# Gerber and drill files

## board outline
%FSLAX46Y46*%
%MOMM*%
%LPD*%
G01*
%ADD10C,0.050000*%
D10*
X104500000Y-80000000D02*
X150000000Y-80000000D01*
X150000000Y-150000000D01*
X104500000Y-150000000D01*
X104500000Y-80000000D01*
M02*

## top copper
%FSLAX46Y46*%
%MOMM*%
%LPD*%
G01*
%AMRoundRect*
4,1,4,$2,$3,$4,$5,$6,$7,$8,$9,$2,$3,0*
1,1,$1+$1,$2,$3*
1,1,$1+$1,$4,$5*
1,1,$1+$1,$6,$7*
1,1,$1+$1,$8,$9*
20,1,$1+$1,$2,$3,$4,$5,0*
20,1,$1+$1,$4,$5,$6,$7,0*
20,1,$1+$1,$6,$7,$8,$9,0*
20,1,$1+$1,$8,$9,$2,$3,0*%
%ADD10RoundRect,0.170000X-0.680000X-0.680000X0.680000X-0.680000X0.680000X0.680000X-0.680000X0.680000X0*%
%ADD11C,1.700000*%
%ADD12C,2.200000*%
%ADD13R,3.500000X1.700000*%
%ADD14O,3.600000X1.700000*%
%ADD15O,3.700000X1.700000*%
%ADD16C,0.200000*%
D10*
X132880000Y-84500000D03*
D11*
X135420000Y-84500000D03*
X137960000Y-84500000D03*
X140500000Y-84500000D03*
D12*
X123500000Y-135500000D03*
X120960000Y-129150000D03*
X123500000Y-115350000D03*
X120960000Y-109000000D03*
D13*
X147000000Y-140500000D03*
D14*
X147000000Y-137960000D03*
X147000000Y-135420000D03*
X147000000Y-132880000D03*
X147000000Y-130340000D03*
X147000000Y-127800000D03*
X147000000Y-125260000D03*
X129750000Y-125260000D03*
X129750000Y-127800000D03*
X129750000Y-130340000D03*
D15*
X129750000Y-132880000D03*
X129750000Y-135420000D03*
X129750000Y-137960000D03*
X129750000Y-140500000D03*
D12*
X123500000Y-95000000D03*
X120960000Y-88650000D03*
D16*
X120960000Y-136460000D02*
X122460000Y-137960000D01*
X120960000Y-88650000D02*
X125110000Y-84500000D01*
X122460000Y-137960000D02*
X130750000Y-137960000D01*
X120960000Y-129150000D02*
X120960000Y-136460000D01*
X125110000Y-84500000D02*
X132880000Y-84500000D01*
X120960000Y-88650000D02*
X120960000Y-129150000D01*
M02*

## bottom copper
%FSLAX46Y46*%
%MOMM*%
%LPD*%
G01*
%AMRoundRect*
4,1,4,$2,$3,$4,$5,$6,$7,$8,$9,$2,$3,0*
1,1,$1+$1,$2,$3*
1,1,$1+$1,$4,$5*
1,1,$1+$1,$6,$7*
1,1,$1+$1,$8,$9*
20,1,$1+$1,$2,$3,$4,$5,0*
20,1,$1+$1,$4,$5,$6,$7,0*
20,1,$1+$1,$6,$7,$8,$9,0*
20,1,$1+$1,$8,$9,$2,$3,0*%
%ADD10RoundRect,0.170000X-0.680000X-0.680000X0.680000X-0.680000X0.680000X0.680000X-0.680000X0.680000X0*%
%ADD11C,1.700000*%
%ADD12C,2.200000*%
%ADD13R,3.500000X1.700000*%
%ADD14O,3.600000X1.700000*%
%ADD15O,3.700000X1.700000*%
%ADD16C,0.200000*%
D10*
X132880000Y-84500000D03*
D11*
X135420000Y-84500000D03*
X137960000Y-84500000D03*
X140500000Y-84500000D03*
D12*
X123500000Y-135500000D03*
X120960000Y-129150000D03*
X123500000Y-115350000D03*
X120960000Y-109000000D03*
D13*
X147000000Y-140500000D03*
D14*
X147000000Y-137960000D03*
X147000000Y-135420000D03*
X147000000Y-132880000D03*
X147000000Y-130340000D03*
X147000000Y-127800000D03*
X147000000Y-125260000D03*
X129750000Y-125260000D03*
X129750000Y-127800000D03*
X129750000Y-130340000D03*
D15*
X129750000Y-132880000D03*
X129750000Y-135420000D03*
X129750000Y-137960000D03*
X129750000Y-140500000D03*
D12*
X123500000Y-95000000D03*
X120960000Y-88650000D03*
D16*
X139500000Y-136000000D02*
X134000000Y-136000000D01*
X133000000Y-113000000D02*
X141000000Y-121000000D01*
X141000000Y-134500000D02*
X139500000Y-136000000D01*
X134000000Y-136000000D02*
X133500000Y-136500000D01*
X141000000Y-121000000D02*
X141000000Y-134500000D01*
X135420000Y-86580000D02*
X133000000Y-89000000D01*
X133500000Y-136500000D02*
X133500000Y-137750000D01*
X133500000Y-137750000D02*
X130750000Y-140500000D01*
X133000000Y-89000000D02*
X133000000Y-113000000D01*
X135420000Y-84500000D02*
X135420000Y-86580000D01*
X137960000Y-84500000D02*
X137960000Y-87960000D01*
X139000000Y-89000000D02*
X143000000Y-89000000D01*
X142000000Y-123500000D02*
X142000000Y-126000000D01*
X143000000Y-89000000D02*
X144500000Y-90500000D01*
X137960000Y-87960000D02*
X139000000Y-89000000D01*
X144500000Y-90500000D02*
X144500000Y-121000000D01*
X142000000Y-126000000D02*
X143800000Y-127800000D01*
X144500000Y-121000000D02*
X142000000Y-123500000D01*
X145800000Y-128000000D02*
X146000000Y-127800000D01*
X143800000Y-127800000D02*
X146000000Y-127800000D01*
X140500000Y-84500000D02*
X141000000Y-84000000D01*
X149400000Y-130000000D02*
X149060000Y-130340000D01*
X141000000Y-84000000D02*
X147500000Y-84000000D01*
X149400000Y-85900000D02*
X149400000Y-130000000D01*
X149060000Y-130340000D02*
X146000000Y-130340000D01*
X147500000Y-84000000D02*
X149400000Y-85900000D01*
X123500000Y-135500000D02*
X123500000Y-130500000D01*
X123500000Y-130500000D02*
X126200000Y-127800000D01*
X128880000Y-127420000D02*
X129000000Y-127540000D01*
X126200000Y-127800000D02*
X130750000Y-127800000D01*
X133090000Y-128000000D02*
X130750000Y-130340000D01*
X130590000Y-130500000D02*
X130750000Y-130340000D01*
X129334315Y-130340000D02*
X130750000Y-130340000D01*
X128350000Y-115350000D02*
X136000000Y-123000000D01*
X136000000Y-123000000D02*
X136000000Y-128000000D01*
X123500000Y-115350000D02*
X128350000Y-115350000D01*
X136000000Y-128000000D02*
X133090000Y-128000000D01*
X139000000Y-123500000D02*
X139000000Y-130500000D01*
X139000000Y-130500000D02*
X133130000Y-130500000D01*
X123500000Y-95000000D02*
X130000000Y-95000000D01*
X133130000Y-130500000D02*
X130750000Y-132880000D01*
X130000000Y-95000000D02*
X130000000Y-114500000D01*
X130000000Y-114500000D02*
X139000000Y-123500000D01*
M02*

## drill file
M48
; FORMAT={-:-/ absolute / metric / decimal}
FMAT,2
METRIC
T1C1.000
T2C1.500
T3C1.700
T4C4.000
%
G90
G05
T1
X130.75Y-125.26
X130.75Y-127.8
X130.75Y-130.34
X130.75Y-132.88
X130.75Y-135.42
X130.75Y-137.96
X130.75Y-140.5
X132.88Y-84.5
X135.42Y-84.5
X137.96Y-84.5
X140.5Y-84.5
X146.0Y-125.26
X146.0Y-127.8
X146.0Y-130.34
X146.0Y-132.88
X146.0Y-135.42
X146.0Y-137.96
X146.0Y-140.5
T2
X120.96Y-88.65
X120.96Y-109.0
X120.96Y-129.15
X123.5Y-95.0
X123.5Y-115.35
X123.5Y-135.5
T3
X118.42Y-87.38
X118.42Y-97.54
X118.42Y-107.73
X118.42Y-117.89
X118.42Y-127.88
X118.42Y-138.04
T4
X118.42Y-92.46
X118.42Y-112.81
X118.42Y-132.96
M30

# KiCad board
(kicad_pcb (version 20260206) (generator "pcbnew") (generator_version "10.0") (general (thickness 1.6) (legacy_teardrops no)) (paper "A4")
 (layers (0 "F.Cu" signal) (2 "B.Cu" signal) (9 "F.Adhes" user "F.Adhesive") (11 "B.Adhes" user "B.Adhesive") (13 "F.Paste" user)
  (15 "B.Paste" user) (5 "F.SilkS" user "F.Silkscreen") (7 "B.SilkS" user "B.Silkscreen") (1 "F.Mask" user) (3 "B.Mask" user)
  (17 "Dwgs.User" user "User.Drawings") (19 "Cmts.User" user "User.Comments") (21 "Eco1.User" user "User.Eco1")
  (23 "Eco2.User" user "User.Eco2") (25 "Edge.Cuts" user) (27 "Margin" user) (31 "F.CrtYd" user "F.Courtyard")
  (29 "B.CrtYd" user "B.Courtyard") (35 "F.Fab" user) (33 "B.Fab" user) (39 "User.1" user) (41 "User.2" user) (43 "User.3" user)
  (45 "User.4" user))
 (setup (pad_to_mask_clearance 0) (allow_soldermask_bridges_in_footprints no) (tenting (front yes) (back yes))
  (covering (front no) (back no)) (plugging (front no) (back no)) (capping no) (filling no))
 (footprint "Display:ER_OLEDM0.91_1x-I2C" (layer "F.Cu") (at 132.88 84.5)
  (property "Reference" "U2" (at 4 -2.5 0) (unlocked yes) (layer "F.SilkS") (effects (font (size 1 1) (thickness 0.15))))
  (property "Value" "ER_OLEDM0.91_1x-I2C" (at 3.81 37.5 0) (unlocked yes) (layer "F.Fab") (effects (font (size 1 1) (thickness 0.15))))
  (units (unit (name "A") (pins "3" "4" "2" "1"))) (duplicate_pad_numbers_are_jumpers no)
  (pad "1" thru_hole roundrect (at 0 0) (size 1.7 1.7) (drill 1) (layers "*.Cu" "*.Mask") (remove_unused_layers no) (roundrect_rratio 0.1)
   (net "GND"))
  (pad "2" thru_hole circle (at 2.54 0) (size 1.7 1.7) (drill 1) (layers "*.Cu" "*.Mask") (remove_unused_layers no) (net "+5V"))
  (pad "3" thru_hole circle (at 5.08 0) (size 1.7 1.7) (drill 1) (layers "*.Cu" "*.Mask") (remove_unused_layers no)
   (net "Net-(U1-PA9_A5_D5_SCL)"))
  (pad "4" thru_hole circle (at 7.62 0) (size 1.7 1.7) (drill 1) (layers "*.Cu" "*.Mask") (remove_unused_layers no)
   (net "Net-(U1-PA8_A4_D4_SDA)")))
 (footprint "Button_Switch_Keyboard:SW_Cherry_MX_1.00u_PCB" (layer "F.Cu") (at 123.5 135.5 -90)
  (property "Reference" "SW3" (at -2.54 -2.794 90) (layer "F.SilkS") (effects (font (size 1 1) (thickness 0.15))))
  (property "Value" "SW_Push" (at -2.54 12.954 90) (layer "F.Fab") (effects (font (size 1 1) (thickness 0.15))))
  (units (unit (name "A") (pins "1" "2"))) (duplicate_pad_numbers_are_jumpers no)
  (pad "" np_thru_hole circle (at -7.62 5.08 270) (size 1.7 1.7) (drill 1.7) (layers "*.Cu" "*.Mask"))
  (pad "" np_thru_hole circle (at -2.54 5.08 270) (size 4 4) (drill 4) (layers "*.Cu" "*.Mask"))
  (pad "" np_thru_hole circle (at 2.54 5.08 270) (size 1.7 1.7) (drill 1.7) (layers "*.Cu" "*.Mask"))
  (pad "1" thru_hole circle (at 0 0 270) (size 2.2 2.2) (drill 1.5) (layers "*.Cu" "*.Mask") (remove_unused_layers no)
   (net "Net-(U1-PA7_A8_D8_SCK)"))
  (pad "2" thru_hole circle (at -6.35 2.54 270) (size 2.2 2.2) (drill 1.5) (layers "*.Cu" "*.Mask") (remove_unused_layers no) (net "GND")))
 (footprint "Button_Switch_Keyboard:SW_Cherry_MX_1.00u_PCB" (layer "F.Cu") (at 123.5 115.35 -90)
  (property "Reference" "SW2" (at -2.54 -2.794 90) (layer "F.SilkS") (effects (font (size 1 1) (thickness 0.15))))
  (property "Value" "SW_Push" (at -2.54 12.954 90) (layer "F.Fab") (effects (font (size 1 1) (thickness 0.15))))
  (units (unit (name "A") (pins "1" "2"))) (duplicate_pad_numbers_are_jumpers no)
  (pad "" np_thru_hole circle (at -7.62 5.08 270) (size 1.7 1.7) (drill 1.7) (layers "*.Cu" "*.Mask"))
  (pad "" np_thru_hole circle (at -2.54 5.08 270) (size 4 4) (drill 4) (layers "*.Cu" "*.Mask"))
  (pad "" np_thru_hole circle (at 2.54 5.08 270) (size 1.7 1.7) (drill 1.7) (layers "*.Cu" "*.Mask"))
  (pad "1" thru_hole circle (at 0 0 270) (size 2.2 2.2) (drill 1.5) (layers "*.Cu" "*.Mask") (remove_unused_layers no)
   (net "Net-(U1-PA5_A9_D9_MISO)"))
  (pad "2" thru_hole circle (at -6.35 2.54 270) (size 2.2 2.2) (drill 1.5) (layers "*.Cu" "*.Mask") (remove_unused_layers no) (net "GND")))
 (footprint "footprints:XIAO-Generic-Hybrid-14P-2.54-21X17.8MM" (layer "F.Cu") (at 138.375 132.88 180)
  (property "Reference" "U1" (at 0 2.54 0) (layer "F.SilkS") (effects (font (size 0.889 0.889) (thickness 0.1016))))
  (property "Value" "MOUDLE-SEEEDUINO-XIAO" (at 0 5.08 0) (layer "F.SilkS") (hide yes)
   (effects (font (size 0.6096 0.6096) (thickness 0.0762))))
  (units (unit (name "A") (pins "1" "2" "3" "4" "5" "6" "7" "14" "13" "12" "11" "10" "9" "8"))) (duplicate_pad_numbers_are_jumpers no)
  (pad "1" thru_hole rect (at -7.625 -7.62 180) (size 3.5 1.7) (drill 1 (offset -1 0)) (layers "*.Cu" "*.Mask") (remove_unused_layers no)
   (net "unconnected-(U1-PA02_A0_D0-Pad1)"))
  (pad "2" thru_hole oval (at -7.625 -5.08 180) (size 3.6 1.7) (drill 1 (offset -1 0)) (layers "*.Cu" "*.Mask") (remove_unused_layers no)
   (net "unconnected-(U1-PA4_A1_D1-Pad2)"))
  (pad "3" thru_hole oval (at -7.625 -2.54 180) (size 3.6 1.7) (drill 1 (offset -1 0)) (layers "*.Cu" "*.Mask") (remove_unused_layers no)
   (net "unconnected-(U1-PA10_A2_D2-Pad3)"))
  (pad "4" thru_hole oval (at -7.625 0 180) (size 3.6 1.7) (drill 1 (offset -1 0)) (layers "*.Cu" "*.Mask") (remove_unused_layers no)
   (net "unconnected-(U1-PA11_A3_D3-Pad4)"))
  (pad "5" thru_hole oval (at -7.625 2.54 180) (size 3.6 1.7) (drill 1 (offset -1 0)) (layers "*.Cu" "*.Mask") (remove_unused_layers no)
   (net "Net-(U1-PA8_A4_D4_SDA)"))
  (pad "6" thru_hole oval (at -7.625 5.08) (size 3.6 1.7) (drill 1 (offset 1 0)) (layers "*.Cu" "*.Mask") (remove_unused_layers no)
   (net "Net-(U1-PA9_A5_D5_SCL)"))
  (pad "7" thru_hole oval (at -7.625 7.62 180) (size 3.6 1.7) (drill 1 (offset -1 0)) (layers "*.Cu" "*.Mask") (remove_unused_layers no)
   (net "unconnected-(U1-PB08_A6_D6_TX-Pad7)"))
  (pad "8" thru_hole oval (at 7.625 7.62 180) (size 3.6 1.7) (drill 1 (offset 1 0)) (layers "*.Cu" "*.Mask") (remove_unused_layers no)
   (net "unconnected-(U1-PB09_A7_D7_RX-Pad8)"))
  (pad "9" thru_hole oval (at 7.625 5.08 180) (size 3.6 1.7) (drill 1 (offset 1 0)) (layers "*.Cu" "*.Mask") (remove_unused_layers no)
   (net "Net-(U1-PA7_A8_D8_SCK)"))
  (pad "10" thru_hole oval (at 7.625 2.54 180) (size 3.6 1.7) (drill 1 (offset 1 0)) (layers "*.Cu" "*.Mask") (remove_unused_layers no)
   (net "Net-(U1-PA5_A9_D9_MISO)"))
  (pad "11" thru_hole oval (at 7.625 0 180) (size 3.7 1.7) (drill 1 (offset 1 0)) (layers "*.Cu" "*.Mask") (remove_unused_layers no)
   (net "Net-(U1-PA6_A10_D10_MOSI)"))
  (pad "12" thru_hole oval (at 7.625 -2.54 180) (size 3.7 1.7) (drill 1 (offset 1 0)) (layers "*.Cu" "*.Mask") (remove_unused_layers no)
   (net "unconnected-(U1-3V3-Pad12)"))
  (pad "13" thru_hole oval (at 7.625 -5.08 180) (size 3.7 1.7) (drill 1 (offset 1 0)) (layers "*.Cu" "*.Mask") (remove_unused_layers no)
   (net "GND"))
  (pad "14" thru_hole oval (at 7.625 -7.62 180) (size 3.7 1.7) (drill 1 (offset 1 0)) (layers "*.Cu" "*.Mask") (remove_unused_layers no)
   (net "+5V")))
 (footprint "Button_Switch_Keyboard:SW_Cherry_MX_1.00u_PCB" (layer "F.Cu") (at 123.5 95 -90)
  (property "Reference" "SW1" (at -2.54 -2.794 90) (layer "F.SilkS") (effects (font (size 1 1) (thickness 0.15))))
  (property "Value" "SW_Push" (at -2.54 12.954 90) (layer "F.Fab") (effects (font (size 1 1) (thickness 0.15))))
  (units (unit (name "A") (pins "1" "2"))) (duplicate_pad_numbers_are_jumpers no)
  (pad "" np_thru_hole circle (at -7.62 5.08 270) (size 1.7 1.7) (drill 1.7) (layers "*.Cu" "*.Mask"))
  (pad "" np_thru_hole circle (at -2.54 5.08 270) (size 4 4) (drill 4) (layers "*.Cu" "*.Mask"))
  (pad "" np_thru_hole circle (at 2.54 5.08 270) (size 1.7 1.7) (drill 1.7) (layers "*.Cu" "*.Mask"))
  (pad "1" thru_hole circle (at 0 0 270) (size 2.2 2.2) (drill 1.5) (layers "*.Cu" "*.Mask") (remove_unused_layers no)
   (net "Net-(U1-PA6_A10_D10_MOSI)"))
  (pad "2" thru_hole circle (at -6.35 2.54 270) (size 2.2 2.2) (drill 1.5) (layers "*.Cu" "*.Mask") (remove_unused_layers no) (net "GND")))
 (gr_rect (start 104.5 80) (end 150 150) (stroke (width 0.05) (type default)) (fill no) (layer "Edge.Cuts"))
 (segment (start 120.96 136.46) (end 122.46 137.96) (width 0.2) (layer "F.Cu") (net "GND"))
 (segment (start 120.96 88.65) (end 125.11 84.5) (width 0.2) (layer "F.Cu") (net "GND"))
 (segment (start 122.46 137.96) (end 130.75 137.96) (width 0.2) (layer "F.Cu") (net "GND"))
 (segment (start 120.96 129.15) (end 120.96 136.46) (width 0.2) (layer "F.Cu") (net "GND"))
 (segment (start 125.11 84.5) (end 132.88 84.5) (width 0.2) (layer "F.Cu") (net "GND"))
 (segment (start 120.96 88.65) (end 120.96 129.15) (width 0.2) (layer "F.Cu") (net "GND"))
 (segment (start 139.5 136) (end 134 136) (width 0.2) (layer "B.Cu") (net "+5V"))
 (segment (start 133 113) (end 141 121) (width 0.2) (layer "B.Cu") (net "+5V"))
 (segment (start 141 134.5) (end 139.5 136) (width 0.2) (layer "B.Cu") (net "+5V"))
 (segment (start 134 136) (end 133.5 136.5) (width 0.2) (layer "B.Cu") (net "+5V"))
 (segment (start 141 121) (end 141 134.5) (width 0.2) (layer "B.Cu") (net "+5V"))
 (segment (start 135.42 86.58) (end 133 89) (width 0.2) (layer "B.Cu") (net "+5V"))
 (segment (start 133.5 136.5) (end 133.5 137.75) (width 0.2) (layer "B.Cu") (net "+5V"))
 (segment (start 133.5 137.75) (end 130.75 140.5) (width 0.2) (layer "B.Cu") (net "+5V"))
 (segment (start 133 89) (end 133 113) (width 0.2) (layer "B.Cu") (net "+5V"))
 (segment (start 135.42 84.5) (end 135.42 86.58) (width 0.2) (layer "B.Cu") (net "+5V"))
 (segment (start 137.96 84.5) (end 137.96 87.96) (width 0.2) (layer "B.Cu") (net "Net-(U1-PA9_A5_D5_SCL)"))
 (segment (start 139 89) (end 143 89) (width 0.2) (layer "B.Cu") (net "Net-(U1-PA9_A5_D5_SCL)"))
 (segment (start 142 123.5) (end 142 126) (width 0.2) (layer "B.Cu") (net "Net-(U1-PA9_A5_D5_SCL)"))
 (segment (start 143 89) (end 144.5 90.5) (width 0.2) (layer "B.Cu") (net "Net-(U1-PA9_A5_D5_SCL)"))
 (segment (start 137.96 87.96) (end 139 89) (width 0.2) (layer "B.Cu") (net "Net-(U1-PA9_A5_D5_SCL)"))
 (segment (start 144.5 90.5) (end 144.5 121) (width 0.2) (layer "B.Cu") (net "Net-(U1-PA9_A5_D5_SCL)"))
 (segment (start 142 126) (end 143.8 127.8) (width 0.2) (layer "B.Cu") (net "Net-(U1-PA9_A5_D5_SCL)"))
 (segment (start 144.5 121) (end 142 123.5) (width 0.2) (layer "B.Cu") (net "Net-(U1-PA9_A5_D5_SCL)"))
 (segment (start 145.8 128) (end 146 127.8) (width 0.2) (layer "B.Cu") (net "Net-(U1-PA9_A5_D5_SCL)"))
 (segment (start 143.8 127.8) (end 146 127.8) (width 0.2) (layer "B.Cu") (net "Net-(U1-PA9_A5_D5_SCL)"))
 (segment (start 140.5 84.5) (end 141 84) (width 0.2) (layer "B.Cu") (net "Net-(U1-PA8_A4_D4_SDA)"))
 (segment (start 149.4 130) (end 149.06 130.34) (width 0.2) (layer "B.Cu") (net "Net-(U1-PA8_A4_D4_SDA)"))
 (segment (start 141 84) (end 147.5 84) (width 0.2) (layer "B.Cu") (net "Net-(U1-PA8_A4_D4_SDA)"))
 (segment (start 149.4 85.9) (end 149.4 130) (width 0.2) (layer "B.Cu") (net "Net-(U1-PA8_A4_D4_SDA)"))
 (segment (start 149.06 130.34) (end 146 130.34) (width 0.2) (layer "B.Cu") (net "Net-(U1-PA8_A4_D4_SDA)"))
 (segment (start 147.5 84) (end 149.4 85.9) (width 0.2) (layer "B.Cu") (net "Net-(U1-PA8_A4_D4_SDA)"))
 (segment (start 123.5 135.5) (end 123.5 130.5) (width 0.2) (layer "B.Cu") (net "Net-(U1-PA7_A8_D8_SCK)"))
 (segment (start 123.5 130.5) (end 126.2 127.8) (width 0.2) (layer "B.Cu") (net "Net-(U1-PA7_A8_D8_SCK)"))
 (segment (start 128.88 127.42) (end 129 127.54) (width 0.2) (layer "B.Cu") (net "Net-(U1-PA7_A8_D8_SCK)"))
 (segment (start 126.2 127.8) (end 130.75 127.8) (width 0.2) (layer "B.Cu") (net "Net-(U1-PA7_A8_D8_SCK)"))
 (segment (start 133.09 128) (end 130.75 130.34) (width 0.2) (layer "B.Cu") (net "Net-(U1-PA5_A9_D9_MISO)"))
 (segment (start 130.59 130.5) (end 130.75 130.34) (width 0.2) (layer "B.Cu") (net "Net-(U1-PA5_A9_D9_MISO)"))
 (segment (start 129.334315 130.34) (end 130.75 130.34) (width 0.2) (layer "B.Cu") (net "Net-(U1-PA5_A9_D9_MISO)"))
 (segment (start 128.35 115.35) (end 136 123) (width 0.2) (layer "B.Cu") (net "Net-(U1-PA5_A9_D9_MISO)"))
 (segment (start 136 123) (end 136 128) (width 0.2) (layer "B.Cu") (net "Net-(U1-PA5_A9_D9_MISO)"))
 (segment (start 123.5 115.35) (end 128.35 115.35) (width 0.2) (layer "B.Cu") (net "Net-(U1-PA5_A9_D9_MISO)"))
 (segment (start 136 128) (end 133.09 128) (width 0.2) (layer "B.Cu") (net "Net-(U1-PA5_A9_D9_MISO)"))
 (segment (start 139 123.5) (end 139 130.5) (width 0.2) (layer "B.Cu") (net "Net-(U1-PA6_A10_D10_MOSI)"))
 (segment (start 139 130.5) (end 133.13 130.5) (width 0.2) (layer "B.Cu") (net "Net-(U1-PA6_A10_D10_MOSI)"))
 (segment (start 123.5 95) (end 130 95) (width 0.2) (layer "B.Cu") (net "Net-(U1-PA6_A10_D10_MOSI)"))
 (segment (start 133.13 130.5) (end 130.75 132.88) (width 0.2) (layer "B.Cu") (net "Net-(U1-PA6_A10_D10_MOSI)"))
 (segment (start 130 95) (end 130 114.5) (width 0.2) (layer "B.Cu") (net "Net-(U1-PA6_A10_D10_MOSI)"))
 (segment (start 130 114.5) (end 139 123.5) (width 0.2) (layer "B.Cu") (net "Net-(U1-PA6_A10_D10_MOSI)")))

